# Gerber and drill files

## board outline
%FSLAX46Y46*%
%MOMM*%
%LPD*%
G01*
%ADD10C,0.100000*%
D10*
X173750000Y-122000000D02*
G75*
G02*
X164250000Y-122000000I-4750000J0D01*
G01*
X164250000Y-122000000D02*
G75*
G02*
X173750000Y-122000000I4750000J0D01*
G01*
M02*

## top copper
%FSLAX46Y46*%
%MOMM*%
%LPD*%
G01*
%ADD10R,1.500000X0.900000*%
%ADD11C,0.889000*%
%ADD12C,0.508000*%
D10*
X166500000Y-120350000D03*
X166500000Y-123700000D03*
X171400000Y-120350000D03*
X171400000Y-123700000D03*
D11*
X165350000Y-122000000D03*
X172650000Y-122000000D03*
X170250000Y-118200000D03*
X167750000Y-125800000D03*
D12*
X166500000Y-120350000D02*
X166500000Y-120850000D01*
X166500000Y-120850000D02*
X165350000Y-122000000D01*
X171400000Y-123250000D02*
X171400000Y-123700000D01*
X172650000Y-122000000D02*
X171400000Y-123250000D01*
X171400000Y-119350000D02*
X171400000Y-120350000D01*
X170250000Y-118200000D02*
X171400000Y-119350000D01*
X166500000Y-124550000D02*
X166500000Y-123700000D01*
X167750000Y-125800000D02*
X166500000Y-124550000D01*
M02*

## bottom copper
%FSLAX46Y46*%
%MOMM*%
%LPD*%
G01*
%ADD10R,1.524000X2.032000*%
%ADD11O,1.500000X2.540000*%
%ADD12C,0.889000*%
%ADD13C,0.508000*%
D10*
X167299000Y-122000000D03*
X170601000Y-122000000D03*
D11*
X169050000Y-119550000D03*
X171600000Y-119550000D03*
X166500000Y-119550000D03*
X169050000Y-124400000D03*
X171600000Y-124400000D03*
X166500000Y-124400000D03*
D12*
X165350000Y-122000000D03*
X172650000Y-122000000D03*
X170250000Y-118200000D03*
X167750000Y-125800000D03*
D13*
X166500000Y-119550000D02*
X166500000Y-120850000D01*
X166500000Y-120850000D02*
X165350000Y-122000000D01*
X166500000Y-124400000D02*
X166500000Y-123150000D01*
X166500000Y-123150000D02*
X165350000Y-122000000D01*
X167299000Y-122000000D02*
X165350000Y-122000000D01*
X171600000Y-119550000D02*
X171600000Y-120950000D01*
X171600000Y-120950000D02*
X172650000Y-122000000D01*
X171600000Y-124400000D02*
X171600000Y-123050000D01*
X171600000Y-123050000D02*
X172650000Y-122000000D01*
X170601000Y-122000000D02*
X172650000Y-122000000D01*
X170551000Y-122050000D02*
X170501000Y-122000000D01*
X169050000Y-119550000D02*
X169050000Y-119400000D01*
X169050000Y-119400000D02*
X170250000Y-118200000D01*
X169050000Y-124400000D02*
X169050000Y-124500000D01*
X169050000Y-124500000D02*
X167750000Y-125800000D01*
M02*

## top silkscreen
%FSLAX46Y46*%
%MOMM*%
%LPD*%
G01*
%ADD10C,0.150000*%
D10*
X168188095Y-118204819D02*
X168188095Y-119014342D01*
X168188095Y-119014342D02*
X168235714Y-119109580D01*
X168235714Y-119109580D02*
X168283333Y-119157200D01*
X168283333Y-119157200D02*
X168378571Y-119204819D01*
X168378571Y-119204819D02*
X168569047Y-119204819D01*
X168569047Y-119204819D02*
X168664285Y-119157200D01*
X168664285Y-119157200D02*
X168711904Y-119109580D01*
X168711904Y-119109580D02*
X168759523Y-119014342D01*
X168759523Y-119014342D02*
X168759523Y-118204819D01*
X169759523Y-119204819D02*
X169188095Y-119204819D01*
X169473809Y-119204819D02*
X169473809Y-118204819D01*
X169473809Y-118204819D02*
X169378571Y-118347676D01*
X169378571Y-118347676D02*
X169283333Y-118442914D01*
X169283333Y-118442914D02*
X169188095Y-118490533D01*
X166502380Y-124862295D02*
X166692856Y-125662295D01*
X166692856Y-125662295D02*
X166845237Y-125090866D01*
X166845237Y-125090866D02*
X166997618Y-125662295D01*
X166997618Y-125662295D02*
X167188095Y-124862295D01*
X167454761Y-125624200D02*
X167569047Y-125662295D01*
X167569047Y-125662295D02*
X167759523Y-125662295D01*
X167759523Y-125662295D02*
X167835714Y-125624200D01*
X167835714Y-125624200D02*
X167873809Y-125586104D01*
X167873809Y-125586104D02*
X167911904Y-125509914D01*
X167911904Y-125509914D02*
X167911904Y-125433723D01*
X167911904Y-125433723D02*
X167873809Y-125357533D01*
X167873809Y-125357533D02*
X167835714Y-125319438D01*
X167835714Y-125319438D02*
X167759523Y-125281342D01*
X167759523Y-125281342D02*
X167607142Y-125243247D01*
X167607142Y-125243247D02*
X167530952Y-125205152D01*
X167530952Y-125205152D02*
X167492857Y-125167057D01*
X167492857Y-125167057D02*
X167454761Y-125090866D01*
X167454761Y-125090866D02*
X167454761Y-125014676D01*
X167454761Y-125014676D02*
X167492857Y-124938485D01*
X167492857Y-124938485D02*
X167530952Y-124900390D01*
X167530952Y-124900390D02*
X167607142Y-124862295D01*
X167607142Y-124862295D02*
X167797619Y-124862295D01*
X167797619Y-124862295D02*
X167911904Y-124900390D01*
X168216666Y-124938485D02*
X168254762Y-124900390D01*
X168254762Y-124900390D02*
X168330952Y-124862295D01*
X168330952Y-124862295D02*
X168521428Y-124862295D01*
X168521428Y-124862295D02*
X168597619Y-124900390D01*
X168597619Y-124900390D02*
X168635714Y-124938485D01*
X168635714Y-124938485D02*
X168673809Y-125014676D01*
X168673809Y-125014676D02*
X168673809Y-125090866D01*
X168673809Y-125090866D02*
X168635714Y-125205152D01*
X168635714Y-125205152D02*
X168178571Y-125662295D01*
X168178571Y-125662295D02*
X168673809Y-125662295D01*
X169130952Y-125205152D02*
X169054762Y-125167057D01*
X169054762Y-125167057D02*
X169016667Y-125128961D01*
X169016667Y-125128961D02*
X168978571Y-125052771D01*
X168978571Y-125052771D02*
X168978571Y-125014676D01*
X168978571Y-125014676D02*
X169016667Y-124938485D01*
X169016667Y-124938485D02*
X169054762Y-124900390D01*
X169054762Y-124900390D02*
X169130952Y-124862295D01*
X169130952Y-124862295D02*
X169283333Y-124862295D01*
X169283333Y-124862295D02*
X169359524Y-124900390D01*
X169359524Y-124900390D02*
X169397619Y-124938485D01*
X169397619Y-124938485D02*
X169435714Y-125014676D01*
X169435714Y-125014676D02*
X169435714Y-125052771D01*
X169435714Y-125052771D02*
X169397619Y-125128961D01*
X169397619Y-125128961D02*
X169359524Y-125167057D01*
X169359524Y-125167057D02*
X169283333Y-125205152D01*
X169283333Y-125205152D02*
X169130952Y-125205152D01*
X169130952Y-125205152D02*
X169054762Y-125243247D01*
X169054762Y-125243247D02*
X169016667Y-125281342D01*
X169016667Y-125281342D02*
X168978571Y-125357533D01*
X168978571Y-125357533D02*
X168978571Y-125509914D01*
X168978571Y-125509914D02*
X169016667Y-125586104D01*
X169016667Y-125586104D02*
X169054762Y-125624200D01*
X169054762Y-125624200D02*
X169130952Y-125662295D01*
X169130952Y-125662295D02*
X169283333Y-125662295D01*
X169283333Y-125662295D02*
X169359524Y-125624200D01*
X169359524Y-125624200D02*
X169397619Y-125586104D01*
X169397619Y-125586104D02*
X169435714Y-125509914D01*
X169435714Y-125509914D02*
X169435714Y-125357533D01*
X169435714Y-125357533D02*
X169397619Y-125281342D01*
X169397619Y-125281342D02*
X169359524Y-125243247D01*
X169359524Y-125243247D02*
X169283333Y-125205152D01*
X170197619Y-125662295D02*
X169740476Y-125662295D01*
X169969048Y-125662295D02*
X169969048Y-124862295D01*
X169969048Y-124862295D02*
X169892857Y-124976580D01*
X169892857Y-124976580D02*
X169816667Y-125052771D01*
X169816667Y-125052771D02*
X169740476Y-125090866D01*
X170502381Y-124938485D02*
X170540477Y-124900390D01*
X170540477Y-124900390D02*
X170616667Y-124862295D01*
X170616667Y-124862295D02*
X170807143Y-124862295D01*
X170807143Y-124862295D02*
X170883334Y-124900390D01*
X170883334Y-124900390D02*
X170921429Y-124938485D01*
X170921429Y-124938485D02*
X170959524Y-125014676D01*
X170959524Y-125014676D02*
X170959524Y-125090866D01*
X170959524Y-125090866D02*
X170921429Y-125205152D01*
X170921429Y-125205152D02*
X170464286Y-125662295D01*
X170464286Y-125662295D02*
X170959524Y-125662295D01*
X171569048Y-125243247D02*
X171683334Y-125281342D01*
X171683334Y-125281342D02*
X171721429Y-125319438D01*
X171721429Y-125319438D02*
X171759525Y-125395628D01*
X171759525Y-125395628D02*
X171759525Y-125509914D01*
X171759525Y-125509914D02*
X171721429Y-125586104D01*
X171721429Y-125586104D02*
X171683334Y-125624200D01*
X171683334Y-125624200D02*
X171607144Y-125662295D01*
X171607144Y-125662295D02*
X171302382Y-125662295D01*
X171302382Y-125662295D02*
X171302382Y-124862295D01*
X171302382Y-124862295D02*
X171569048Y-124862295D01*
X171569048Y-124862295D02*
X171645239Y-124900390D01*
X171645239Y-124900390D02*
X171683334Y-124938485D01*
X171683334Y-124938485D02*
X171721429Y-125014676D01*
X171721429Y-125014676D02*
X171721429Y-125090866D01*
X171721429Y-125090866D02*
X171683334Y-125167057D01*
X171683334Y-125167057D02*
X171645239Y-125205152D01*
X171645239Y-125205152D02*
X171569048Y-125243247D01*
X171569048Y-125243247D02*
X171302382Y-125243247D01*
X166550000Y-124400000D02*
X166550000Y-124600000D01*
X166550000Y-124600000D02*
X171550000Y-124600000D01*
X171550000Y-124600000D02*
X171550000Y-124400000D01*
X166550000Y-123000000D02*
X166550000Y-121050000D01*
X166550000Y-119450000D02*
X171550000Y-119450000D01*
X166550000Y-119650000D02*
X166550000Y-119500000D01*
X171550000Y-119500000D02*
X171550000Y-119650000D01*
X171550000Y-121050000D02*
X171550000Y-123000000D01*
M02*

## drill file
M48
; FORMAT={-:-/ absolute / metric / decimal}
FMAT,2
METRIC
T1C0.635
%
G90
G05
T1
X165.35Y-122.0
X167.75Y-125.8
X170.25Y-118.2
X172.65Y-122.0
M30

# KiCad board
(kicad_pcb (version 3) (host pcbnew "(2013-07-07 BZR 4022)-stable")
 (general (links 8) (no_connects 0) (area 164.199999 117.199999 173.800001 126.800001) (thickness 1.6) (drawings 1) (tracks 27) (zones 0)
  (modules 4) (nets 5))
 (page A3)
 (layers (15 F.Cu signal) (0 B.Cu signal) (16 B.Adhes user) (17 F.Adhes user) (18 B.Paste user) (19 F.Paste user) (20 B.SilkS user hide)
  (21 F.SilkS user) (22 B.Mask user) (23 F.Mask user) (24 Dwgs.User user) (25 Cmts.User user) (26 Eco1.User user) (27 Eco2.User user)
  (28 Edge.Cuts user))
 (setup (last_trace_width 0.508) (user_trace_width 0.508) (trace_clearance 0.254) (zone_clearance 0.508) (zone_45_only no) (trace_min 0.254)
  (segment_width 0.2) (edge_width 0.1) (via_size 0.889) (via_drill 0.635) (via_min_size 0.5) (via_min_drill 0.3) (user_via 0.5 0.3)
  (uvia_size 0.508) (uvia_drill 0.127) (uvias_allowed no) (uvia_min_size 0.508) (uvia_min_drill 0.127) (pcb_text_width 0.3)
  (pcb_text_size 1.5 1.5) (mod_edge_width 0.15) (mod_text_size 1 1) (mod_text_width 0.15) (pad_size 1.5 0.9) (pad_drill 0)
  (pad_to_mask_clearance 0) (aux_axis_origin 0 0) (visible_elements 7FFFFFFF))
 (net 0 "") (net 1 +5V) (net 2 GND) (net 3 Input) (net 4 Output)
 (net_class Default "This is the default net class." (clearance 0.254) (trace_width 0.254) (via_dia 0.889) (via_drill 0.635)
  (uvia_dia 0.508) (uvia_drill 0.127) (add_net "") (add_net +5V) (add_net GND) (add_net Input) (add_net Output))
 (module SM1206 (layer B.Cu) (at 168.95 122)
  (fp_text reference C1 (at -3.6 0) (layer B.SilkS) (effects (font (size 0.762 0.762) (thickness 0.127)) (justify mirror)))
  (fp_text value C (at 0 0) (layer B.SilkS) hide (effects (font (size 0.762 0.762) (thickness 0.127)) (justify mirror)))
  (pad 1 smd rect (at -1.651 0) (size 1.524 2.032) (layers B.Cu B.Paste B.Mask) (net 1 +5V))
  (pad 2 smd rect (at 1.651 0) (size 1.524 2.032) (layers B.Cu B.Paste B.Mask) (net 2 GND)))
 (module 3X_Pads (layer B.Cu) (at 169.05 119.55 270)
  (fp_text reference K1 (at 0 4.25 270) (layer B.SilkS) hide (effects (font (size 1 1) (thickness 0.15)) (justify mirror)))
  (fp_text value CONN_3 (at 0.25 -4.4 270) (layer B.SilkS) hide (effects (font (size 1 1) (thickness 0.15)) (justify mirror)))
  (pad 2 smd oval (at 0 0 270) (size 2.54 1.5) (layers B.Cu B.Paste B.Mask) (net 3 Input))
  (pad 3 smd oval (at 0 -2.55 270) (size 2.54 1.5) (layers B.Cu B.Paste B.Mask) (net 2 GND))
  (pad 1 smd oval (at 0 2.55 270) (size 2.54 1.5) (layers B.Cu B.Paste B.Mask) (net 1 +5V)))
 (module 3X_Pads (layer B.Cu) (at 169.05 124.4 270)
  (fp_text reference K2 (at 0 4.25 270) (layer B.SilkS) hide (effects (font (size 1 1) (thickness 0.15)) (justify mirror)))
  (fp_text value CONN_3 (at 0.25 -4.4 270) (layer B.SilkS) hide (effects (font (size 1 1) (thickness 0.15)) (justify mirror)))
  (pad 2 smd oval (at 0 0 270) (size 2.54 1.5) (layers B.Cu B.Paste B.Mask) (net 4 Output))
  (pad 3 smd oval (at 0 -2.55 270) (size 2.54 1.5) (layers B.Cu B.Paste B.Mask) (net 2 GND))
  (pad 1 smd oval (at 0 2.55 270) (size 2.54 1.5) (layers B.Cu B.Paste B.Mask) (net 1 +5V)))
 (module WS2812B (layer F.Cu) (at 166.5 120.35)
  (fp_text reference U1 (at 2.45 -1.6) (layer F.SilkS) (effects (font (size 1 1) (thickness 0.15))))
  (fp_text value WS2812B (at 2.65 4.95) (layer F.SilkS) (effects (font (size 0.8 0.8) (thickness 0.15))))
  (fp_line (start 0.05 4.05) (end 0.05 4.25) (layer F.SilkS) (width 0.15))
  (fp_line (start 0.05 4.25) (end 5.05 4.25) (layer F.SilkS) (width 0.15))
  (fp_line (start 5.05 4.25) (end 5.05 4.05) (layer F.SilkS) (width 0.15))
  (fp_line (start 0.05 2.65) (end 0.05 0.7) (layer F.SilkS) (width 0.15))
  (fp_line (start 0.05 -0.9) (end 5.05 -0.9) (layer F.SilkS) (width 0.15))
  (fp_line (start 0.05 -0.7) (end 0.05 -0.85) (layer F.SilkS) (width 0.15))
  (fp_line (start 5.05 -0.85) (end 5.05 -0.7) (layer F.SilkS) (width 0.15))
  (fp_line (start 5.05 0.7) (end 5.05 2.65) (layer F.SilkS) (width 0.15))
  (pad 1 smd rect (at 0 0) (size 1.5 0.9) (layers F.Cu F.Paste F.Mask) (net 1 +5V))
  (pad 2 smd rect (at 0 3.35) (size 1.5 0.9) (layers F.Cu F.Paste F.Mask) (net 4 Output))
  (pad 4 smd rect (at 4.9 0) (size 1.5 0.9) (layers F.Cu F.Paste F.Mask) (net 3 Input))
  (pad 3 smd rect (at 4.9 3.35) (size 1.5 0.9) (layers F.Cu F.Paste F.Mask) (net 2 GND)))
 (gr_circle (center 169 122) (end 164.25 122) (layer Edge.Cuts) (width 0.1))
 (segment (start 166.5 119.55) (end 166.5 120.85) (width 0.508) (layer B.Cu) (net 1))
 (segment (start 166.5 120.85) (end 165.35 122) (width 0.508) (layer B.Cu) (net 1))
 (segment (start 166.5 124.4) (end 166.5 123.15) (width 0.508) (layer B.Cu) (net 1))
 (segment (start 166.5 123.15) (end 165.35 122) (width 0.508) (layer B.Cu) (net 1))
 (via (at 165.35 122) (size 0.889) (layers F.Cu B.Cu) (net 1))
 (segment (start 166.5 120.35) (end 166.5 120.85) (width 0.508) (layer F.Cu) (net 1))
 (segment (start 166.5 120.85) (end 165.35 122) (width 0.508) (layer F.Cu) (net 1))
 (segment (start 167.299 122) (end 165.35 122) (width 0.508) (layer B.Cu) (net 1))
 (segment (start 171.6 119.55) (end 171.6 120.95) (width 0.508) (layer B.Cu) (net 2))
 (segment (start 171.6 120.95) (end 172.65 122) (width 0.508) (layer B.Cu) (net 2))
 (segment (start 171.6 124.4) (end 171.6 123.05) (width 0.508) (layer B.Cu) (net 2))
 (segment (start 171.6 123.05) (end 172.65 122) (width 0.508) (layer B.Cu) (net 2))
 (segment (start 170.601 122) (end 172.65 122) (width 0.508) (layer B.Cu) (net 2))
 (segment (start 171.4 123.25) (end 171.4 123.7) (width 0.508) (layer F.Cu) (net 2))
 (segment (start 172.65 122) (end 171.4 123.25) (width 0.508) (layer F.Cu) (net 2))
 (via (at 172.65 122) (size 0.889) (layers F.Cu B.Cu) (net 2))
 (segment (start 170.551 122.05) (end 170.501 122) (width 0.508) (layer B.Cu) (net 2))
 (segment (start 169.05 119.55) (end 169.05 119.4) (width 0.508) (layer B.Cu) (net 3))
 (segment (start 171.4 119.35) (end 171.4 120.35) (width 0.508) (layer F.Cu) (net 3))
 (segment (start 170.25 118.2) (end 171.4 119.35) (width 0.508) (layer F.Cu) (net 3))
 (via (at 170.25 118.2) (size 0.889) (layers F.Cu B.Cu) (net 3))
 (segment (start 169.05 119.4) (end 170.25 118.2) (width 0.508) (layer B.Cu) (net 3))
 (segment (start 169.05 124.4) (end 169.05 124.5) (width 0.508) (layer B.Cu) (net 4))
 (segment (start 166.5 124.55) (end 166.5 123.7) (width 0.508) (layer F.Cu) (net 4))
 (segment (start 167.75 125.8) (end 166.5 124.55) (width 0.508) (layer F.Cu) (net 4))
 (via (at 167.75 125.8) (size 0.889) (layers F.Cu B.Cu) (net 4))
 (segment (start 169.05 124.5) (end 167.75 125.8) (width 0.508) (layer B.Cu) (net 4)))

